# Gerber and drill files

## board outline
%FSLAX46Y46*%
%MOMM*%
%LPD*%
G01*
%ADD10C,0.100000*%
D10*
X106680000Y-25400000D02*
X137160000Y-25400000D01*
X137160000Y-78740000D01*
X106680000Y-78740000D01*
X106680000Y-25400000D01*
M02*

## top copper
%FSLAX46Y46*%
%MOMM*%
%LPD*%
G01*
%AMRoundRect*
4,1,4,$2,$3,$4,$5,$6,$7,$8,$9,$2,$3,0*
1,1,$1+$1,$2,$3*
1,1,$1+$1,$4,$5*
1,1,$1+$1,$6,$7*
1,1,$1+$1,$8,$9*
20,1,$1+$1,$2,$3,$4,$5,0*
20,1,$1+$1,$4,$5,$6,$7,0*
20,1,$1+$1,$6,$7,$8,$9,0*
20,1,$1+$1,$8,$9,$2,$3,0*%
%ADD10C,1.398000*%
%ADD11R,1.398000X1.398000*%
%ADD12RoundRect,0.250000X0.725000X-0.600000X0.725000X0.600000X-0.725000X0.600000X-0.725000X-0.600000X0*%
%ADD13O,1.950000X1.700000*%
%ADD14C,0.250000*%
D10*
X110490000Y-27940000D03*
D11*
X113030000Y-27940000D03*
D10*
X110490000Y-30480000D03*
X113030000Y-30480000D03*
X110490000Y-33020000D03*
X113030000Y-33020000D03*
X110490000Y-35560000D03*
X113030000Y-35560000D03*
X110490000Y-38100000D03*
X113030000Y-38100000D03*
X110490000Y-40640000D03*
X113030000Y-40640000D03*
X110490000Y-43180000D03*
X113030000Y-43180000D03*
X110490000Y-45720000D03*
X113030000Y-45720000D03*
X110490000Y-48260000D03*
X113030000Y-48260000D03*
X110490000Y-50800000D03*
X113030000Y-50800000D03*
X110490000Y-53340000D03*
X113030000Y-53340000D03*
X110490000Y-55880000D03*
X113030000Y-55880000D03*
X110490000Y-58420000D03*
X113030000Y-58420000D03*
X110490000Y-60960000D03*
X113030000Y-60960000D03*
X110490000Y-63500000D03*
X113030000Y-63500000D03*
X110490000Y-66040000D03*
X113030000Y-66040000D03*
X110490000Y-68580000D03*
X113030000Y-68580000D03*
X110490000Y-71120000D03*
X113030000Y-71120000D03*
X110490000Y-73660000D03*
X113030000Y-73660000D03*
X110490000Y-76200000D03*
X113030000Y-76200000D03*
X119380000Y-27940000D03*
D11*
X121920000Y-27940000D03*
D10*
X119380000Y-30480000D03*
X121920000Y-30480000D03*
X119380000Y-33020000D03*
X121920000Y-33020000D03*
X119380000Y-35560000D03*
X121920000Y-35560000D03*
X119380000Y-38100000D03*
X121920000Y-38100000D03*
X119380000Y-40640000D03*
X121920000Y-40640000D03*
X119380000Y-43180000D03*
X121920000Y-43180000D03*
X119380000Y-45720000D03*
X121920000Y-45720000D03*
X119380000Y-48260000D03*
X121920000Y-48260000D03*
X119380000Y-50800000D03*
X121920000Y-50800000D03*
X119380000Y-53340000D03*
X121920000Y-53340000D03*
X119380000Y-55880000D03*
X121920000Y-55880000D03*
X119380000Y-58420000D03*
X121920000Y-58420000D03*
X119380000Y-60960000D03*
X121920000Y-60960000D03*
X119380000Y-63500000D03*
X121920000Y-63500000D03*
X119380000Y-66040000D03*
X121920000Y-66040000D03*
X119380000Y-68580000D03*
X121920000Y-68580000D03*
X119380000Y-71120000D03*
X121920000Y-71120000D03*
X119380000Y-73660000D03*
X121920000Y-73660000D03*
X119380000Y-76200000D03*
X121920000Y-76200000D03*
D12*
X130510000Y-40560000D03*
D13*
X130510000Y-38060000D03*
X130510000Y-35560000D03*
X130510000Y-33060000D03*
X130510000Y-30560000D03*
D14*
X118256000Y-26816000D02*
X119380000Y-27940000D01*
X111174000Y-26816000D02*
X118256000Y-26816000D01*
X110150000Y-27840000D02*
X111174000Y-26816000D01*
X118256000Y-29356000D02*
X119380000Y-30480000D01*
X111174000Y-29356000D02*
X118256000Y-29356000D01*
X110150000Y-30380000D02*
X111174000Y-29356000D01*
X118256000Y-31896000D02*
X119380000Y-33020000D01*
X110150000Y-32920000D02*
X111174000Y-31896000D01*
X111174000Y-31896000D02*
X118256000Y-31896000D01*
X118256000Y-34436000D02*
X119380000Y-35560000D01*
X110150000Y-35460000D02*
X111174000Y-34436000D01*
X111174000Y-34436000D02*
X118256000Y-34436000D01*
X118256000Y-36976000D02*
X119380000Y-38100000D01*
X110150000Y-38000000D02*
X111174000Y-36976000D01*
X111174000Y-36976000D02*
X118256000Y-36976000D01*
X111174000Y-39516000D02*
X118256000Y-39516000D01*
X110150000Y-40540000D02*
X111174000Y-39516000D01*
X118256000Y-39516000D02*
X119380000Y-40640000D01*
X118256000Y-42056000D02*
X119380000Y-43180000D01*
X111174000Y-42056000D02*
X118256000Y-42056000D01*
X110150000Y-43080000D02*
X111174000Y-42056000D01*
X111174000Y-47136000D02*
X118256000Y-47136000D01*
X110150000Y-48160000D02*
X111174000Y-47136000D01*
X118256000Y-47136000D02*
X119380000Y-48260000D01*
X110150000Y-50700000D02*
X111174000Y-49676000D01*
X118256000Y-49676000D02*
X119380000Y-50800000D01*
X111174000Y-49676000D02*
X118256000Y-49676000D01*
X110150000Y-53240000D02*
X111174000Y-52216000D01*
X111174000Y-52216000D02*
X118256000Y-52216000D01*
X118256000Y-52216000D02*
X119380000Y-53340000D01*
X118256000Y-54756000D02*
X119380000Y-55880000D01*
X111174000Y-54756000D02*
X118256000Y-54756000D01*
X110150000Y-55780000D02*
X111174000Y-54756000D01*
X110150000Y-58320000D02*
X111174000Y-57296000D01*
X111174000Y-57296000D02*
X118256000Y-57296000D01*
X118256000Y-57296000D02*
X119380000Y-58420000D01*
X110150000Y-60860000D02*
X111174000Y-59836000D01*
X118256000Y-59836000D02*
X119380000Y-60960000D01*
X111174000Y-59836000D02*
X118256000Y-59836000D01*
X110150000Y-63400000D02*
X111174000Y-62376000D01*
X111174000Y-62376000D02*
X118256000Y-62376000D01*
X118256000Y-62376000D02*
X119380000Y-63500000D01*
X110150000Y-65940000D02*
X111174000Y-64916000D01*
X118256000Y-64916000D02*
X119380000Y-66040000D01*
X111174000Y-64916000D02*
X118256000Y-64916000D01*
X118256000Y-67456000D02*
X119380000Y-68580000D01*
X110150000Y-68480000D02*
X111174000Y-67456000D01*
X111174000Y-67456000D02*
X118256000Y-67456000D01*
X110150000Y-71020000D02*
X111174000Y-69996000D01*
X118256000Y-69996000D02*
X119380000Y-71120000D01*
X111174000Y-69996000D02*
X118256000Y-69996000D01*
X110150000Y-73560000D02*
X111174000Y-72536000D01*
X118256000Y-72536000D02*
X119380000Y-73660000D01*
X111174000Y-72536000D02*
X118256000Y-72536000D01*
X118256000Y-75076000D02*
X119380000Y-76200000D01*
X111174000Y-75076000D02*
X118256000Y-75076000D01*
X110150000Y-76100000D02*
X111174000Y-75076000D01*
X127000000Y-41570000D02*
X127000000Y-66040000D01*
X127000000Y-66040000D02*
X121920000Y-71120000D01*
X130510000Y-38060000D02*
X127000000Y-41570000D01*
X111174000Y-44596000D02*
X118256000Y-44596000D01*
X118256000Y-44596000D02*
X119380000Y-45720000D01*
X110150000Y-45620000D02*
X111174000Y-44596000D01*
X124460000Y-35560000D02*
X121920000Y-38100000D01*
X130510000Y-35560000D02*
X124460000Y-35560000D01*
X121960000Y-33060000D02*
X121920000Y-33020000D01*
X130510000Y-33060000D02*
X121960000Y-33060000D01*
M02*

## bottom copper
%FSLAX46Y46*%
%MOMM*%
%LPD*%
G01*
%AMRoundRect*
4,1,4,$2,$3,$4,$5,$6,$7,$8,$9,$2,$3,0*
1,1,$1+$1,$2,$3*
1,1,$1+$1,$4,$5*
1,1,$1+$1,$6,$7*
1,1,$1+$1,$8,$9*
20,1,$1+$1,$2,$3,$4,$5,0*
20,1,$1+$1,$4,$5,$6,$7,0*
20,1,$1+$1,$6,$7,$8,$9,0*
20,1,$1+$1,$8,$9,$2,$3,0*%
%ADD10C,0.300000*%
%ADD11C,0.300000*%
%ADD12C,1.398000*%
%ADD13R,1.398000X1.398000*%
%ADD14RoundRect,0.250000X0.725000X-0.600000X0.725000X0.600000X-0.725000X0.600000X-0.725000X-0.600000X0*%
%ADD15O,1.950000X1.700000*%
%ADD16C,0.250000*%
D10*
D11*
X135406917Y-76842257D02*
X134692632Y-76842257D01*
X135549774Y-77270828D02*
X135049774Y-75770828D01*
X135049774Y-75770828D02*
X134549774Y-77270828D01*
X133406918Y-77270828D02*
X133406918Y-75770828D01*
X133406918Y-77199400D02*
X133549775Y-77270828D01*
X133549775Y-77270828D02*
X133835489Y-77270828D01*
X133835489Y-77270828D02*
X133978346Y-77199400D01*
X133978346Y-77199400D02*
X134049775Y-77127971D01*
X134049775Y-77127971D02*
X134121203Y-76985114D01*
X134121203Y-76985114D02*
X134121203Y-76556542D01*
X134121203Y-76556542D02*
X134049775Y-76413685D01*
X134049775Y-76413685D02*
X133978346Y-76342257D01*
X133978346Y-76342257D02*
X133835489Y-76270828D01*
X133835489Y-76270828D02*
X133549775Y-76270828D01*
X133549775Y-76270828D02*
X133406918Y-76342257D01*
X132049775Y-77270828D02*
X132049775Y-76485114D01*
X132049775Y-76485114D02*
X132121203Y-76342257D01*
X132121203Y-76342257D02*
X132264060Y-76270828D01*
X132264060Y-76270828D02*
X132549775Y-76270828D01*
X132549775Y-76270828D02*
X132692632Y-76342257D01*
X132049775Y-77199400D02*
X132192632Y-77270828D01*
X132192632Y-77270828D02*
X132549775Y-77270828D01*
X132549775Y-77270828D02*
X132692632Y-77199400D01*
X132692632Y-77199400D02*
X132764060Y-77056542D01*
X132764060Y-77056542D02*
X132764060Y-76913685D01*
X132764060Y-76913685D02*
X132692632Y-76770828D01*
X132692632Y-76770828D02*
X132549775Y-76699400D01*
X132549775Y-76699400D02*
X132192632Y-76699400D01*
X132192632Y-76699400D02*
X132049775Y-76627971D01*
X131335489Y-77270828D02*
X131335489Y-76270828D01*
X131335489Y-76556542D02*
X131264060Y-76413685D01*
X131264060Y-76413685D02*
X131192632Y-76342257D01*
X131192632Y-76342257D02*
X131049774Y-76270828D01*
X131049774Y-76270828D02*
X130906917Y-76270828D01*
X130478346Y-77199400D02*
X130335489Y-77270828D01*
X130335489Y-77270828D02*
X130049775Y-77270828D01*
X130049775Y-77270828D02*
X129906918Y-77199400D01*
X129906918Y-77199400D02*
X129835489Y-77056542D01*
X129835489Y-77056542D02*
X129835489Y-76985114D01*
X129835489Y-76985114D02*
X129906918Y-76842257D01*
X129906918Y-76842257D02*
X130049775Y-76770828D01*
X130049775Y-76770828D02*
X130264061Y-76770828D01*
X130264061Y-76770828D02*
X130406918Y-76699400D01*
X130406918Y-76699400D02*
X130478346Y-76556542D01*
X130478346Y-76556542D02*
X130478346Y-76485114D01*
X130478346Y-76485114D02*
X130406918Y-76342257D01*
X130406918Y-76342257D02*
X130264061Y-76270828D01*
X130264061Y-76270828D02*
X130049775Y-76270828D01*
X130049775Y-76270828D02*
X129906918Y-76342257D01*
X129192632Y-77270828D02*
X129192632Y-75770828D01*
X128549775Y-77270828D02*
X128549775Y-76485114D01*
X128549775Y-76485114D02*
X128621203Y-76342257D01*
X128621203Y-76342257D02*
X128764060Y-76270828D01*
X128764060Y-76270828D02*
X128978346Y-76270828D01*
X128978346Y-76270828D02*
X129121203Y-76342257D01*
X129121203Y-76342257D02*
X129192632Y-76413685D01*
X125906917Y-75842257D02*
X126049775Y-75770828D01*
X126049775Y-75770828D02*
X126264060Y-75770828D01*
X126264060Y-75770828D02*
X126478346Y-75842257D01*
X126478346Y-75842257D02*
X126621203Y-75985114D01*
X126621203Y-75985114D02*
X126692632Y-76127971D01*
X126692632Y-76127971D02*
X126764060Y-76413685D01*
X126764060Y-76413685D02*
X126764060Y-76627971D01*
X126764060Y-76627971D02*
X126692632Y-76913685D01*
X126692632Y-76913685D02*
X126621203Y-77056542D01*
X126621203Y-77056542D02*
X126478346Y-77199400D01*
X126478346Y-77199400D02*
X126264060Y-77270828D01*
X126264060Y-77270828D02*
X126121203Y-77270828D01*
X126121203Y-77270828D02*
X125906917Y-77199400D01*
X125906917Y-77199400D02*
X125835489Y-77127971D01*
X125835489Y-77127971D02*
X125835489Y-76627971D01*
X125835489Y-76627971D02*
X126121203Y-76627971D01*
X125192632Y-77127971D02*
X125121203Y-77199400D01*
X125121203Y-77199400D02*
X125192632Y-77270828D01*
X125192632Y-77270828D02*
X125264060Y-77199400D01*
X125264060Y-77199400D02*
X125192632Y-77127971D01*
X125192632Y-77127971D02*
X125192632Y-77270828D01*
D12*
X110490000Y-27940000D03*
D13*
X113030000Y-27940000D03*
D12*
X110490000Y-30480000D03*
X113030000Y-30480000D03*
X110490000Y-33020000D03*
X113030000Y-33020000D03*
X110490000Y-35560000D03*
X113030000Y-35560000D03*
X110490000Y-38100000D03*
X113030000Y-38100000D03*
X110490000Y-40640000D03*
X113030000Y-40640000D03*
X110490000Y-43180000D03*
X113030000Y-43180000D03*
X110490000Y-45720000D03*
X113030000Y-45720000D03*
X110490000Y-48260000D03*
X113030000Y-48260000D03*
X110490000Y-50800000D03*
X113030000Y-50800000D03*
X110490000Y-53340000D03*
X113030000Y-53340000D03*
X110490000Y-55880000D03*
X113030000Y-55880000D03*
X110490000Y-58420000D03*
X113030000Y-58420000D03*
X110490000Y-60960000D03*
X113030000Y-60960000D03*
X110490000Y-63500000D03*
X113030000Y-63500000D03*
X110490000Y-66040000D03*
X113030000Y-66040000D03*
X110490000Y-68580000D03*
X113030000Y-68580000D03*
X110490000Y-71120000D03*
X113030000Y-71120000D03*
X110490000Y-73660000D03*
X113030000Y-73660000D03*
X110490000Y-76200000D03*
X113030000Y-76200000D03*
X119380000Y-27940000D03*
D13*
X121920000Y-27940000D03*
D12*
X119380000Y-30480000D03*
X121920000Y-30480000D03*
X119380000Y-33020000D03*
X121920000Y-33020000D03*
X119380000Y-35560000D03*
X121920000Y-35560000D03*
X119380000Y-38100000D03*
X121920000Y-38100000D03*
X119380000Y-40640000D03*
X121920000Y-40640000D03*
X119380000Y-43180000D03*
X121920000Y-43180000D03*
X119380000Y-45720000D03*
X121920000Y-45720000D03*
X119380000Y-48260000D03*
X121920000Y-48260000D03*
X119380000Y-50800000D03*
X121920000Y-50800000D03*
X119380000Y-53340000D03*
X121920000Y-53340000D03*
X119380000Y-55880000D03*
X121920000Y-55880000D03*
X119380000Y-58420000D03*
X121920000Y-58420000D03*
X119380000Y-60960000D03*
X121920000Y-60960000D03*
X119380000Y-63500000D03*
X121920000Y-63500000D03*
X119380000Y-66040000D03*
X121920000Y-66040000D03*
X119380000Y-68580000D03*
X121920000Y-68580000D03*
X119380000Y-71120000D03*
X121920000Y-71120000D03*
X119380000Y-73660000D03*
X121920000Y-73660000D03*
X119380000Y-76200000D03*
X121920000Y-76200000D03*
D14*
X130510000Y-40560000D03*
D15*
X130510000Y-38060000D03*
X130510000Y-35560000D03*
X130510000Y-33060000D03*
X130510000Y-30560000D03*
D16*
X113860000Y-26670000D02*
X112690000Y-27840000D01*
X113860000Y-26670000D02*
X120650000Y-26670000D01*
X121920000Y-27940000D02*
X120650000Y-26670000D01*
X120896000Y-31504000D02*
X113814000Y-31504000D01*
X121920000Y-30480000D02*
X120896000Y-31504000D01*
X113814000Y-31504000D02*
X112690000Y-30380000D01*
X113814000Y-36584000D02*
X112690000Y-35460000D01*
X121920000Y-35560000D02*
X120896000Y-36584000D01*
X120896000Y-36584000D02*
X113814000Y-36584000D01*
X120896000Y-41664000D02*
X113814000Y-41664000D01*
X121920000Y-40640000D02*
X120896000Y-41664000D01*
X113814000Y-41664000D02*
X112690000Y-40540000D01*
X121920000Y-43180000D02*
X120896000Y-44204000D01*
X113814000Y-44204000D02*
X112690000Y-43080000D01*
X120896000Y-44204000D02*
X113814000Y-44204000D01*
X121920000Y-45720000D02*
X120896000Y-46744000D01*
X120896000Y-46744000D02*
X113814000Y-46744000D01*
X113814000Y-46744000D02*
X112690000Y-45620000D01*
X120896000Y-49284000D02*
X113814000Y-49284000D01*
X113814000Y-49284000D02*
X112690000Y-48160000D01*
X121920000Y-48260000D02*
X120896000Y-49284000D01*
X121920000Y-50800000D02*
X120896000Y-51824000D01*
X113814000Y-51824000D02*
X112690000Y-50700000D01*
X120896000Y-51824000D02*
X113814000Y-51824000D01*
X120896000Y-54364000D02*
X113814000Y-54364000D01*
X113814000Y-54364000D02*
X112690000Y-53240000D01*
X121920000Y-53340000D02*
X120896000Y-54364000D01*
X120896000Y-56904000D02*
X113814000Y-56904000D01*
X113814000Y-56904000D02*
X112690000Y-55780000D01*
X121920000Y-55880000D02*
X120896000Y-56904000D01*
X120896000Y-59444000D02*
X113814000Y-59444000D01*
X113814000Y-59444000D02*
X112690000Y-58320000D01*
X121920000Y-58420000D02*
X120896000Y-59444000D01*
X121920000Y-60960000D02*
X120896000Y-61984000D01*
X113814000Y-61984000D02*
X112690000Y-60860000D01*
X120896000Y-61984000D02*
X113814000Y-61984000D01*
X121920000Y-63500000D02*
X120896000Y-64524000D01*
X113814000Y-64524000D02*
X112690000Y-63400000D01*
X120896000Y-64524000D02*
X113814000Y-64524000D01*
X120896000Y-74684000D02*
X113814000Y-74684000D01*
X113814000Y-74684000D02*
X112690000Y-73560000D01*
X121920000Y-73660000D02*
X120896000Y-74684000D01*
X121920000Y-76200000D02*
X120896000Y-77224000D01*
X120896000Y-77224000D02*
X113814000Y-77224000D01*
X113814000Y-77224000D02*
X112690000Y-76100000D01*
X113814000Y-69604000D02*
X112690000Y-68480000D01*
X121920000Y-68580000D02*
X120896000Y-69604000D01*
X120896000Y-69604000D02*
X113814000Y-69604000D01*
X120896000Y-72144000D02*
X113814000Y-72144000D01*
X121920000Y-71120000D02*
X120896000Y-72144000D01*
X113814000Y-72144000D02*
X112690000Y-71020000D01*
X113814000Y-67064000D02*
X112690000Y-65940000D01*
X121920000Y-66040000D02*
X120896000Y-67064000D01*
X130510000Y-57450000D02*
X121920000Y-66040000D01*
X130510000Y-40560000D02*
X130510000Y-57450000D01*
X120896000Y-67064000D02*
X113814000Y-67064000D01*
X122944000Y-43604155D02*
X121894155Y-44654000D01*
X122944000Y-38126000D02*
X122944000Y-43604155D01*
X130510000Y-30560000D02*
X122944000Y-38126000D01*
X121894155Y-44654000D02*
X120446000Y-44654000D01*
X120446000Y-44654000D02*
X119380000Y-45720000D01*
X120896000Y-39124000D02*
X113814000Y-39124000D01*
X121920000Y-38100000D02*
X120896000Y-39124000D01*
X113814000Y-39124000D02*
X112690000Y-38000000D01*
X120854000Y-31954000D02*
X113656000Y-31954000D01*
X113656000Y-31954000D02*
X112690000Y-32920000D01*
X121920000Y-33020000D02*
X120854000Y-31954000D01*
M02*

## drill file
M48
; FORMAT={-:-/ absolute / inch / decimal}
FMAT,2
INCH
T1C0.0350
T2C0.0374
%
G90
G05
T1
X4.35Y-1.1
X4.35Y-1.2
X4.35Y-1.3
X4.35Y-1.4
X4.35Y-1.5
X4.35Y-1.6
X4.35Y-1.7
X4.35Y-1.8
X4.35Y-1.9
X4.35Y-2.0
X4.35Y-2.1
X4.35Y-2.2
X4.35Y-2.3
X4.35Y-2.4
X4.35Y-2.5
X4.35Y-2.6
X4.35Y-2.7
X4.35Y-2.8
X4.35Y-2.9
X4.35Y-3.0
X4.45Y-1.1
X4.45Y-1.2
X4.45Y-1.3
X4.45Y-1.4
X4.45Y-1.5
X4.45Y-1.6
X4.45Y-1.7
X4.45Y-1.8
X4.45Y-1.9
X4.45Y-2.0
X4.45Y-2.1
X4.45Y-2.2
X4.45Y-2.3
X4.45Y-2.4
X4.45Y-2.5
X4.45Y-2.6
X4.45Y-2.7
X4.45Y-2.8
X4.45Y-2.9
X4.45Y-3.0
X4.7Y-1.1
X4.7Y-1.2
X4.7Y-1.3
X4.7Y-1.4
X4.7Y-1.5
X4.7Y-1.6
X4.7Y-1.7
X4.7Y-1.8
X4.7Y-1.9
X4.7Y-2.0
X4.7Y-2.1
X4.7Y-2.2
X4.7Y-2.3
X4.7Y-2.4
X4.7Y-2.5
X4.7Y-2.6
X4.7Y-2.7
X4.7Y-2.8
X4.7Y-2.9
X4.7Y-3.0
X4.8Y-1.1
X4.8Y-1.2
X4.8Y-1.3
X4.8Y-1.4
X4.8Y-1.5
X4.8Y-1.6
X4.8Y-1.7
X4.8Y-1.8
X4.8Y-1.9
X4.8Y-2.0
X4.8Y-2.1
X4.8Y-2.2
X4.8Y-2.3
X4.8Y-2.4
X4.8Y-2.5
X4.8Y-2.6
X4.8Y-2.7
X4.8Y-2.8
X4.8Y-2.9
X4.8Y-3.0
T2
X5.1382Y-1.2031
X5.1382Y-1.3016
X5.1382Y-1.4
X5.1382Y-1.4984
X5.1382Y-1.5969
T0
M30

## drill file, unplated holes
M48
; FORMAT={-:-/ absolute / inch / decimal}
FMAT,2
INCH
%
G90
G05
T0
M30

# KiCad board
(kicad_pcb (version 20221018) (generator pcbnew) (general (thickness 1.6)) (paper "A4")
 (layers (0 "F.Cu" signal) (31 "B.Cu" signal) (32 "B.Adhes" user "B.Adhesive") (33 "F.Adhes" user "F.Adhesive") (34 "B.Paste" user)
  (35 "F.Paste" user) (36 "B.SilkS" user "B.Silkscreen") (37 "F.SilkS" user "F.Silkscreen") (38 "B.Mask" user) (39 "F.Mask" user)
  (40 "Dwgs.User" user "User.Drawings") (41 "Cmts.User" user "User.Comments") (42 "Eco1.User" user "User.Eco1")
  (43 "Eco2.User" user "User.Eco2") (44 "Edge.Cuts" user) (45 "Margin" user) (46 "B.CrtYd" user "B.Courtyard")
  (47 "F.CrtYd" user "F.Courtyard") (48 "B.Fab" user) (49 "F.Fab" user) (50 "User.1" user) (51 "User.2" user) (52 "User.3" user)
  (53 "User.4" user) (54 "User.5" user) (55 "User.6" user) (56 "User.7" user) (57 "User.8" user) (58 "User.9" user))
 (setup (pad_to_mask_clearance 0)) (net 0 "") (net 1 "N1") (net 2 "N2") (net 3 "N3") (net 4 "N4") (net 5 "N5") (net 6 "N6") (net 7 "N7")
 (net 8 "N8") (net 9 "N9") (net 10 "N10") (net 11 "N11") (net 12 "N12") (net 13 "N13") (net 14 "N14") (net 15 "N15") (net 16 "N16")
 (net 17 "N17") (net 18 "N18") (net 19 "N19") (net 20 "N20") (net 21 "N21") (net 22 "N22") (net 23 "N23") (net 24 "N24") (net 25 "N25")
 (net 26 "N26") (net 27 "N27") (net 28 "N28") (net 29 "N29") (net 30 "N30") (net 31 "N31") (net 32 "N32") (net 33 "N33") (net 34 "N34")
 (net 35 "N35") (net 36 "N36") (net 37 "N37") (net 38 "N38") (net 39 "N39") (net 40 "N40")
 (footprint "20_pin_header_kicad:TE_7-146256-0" (layer "F.Cu") (at 111.76 52.07 -90)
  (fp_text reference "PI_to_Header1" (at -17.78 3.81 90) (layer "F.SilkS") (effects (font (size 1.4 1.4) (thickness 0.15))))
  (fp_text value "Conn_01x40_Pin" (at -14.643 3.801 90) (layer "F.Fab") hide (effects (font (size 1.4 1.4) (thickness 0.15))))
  (pad "1" thru_hole circle (at -24.13 1.27 270) (size 1.398 1.398) (drill 0.89) (layers "*.Cu" "*.Mask") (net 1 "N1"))
  (pad "2" thru_hole rect (at -24.13 -1.27 270) (size 1.398 1.398) (drill 0.89) (layers "*.Cu" "*.Mask") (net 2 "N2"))
  (pad "3" thru_hole circle (at -21.59 1.27 270) (size 1.398 1.398) (drill 0.89) (layers "*.Cu" "*.Mask") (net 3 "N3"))
  (pad "4" thru_hole circle (at -21.59 -1.27 270) (size 1.398 1.398) (drill 0.89) (layers "*.Cu" "*.Mask") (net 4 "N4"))
  (pad "5" thru_hole circle (at -19.05 1.27 270) (size 1.398 1.398) (drill 0.89) (layers "*.Cu" "*.Mask") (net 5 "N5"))
  (pad "6" thru_hole circle (at -19.05 -1.27 270) (size 1.398 1.398) (drill 0.89) (layers "*.Cu" "*.Mask") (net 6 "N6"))
  (pad "7" thru_hole circle (at -16.51 1.27 270) (size 1.398 1.398) (drill 0.89) (layers "*.Cu" "*.Mask") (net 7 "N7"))
  (pad "8" thru_hole circle (at -16.51 -1.27 270) (size 1.398 1.398) (drill 0.89) (layers "*.Cu" "*.Mask") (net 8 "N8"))
  (pad "9" thru_hole circle (at -13.97 1.27 270) (size 1.398 1.398) (drill 0.89) (layers "*.Cu" "*.Mask") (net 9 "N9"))
  (pad "10" thru_hole circle (at -13.97 -1.27 270) (size 1.398 1.398) (drill 0.89) (layers "*.Cu" "*.Mask") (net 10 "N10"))
  (pad "11" thru_hole circle (at -11.43 1.27 270) (size 1.398 1.398) (drill 0.89) (layers "*.Cu" "*.Mask") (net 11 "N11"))
  (pad "12" thru_hole circle (at -11.43 -1.27 270) (size 1.398 1.398) (drill 0.89) (layers "*.Cu" "*.Mask") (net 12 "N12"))
  (pad "13" thru_hole circle (at -8.89 1.27 270) (size 1.398 1.398) (drill 0.89) (layers "*.Cu" "*.Mask") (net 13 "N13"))
  (pad "14" thru_hole circle (at -8.89 -1.27 270) (size 1.398 1.398) (drill 0.89) (layers "*.Cu" "*.Mask") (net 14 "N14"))
  (pad "15" thru_hole circle (at -6.35 1.27 270) (size 1.398 1.398) (drill 0.89) (layers "*.Cu" "*.Mask") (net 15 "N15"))
  (pad "16" thru_hole circle (at -6.35 -1.27 270) (size 1.398 1.398) (drill 0.89) (layers "*.Cu" "*.Mask") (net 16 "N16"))
  (pad "17" thru_hole circle (at -3.81 1.27 270) (size 1.398 1.398) (drill 0.89) (layers "*.Cu" "*.Mask") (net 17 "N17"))
  (pad "18" thru_hole circle (at -3.81 -1.27 270) (size 1.398 1.398) (drill 0.89) (layers "*.Cu" "*.Mask") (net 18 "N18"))
  (pad "19" thru_hole circle (at -1.27 1.27 270) (size 1.398 1.398) (drill 0.89) (layers "*.Cu" "*.Mask") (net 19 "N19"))
  (pad "20" thru_hole circle (at -1.27 -1.27 270) (size 1.398 1.398) (drill 0.89) (layers "*.Cu" "*.Mask") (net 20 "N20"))
  (pad "21" thru_hole circle (at 1.27 1.27 270) (size 1.398 1.398) (drill 0.89) (layers "*.Cu" "*.Mask") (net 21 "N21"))
  (pad "22" thru_hole circle (at 1.27 -1.27 270) (size 1.398 1.398) (drill 0.89) (layers "*.Cu" "*.Mask") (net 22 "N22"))
  (pad "23" thru_hole circle (at 3.81 1.27 270) (size 1.398 1.398) (drill 0.89) (layers "*.Cu" "*.Mask") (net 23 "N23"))
  (pad "24" thru_hole circle (at 3.81 -1.27 270) (size 1.398 1.398) (drill 0.89) (layers "*.Cu" "*.Mask") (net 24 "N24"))
  (pad "25" thru_hole circle (at 6.35 1.27 270) (size 1.398 1.398) (drill 0.89) (layers "*.Cu" "*.Mask") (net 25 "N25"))
  (pad "26" thru_hole circle (at 6.35 -1.27 270) (size 1.398 1.398) (drill 0.89) (layers "*.Cu" "*.Mask") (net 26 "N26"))
  (pad "27" thru_hole circle (at 8.89 1.27 270) (size 1.398 1.398) (drill 0.89) (layers "*.Cu" "*.Mask") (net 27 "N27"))
  (pad "28" thru_hole circle (at 8.89 -1.27 270) (size 1.398 1.398) (drill 0.89) (layers "*.Cu" "*.Mask") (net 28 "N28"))
  (pad "29" thru_hole circle (at 11.43 1.27 270) (size 1.398 1.398) (drill 0.89) (layers "*.Cu" "*.Mask") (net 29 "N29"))
  (pad "30" thru_hole circle (at 11.43 -1.27 270) (size 1.398 1.398) (drill 0.89) (layers "*.Cu" "*.Mask") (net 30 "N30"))
  (pad "31" thru_hole circle (at 13.97 1.27 270) (size 1.398 1.398) (drill 0.89) (layers "*.Cu" "*.Mask") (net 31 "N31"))
  (pad "32" thru_hole circle (at 13.97 -1.27 270) (size 1.398 1.398) (drill 0.89) (layers "*.Cu" "*.Mask") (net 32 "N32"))
  (pad "33" thru_hole circle (at 16.51 1.27 270) (size 1.398 1.398) (drill 0.89) (layers "*.Cu" "*.Mask") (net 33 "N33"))
  (pad "34" thru_hole circle (at 16.51 -1.27 270) (size 1.398 1.398) (drill 0.89) (layers "*.Cu" "*.Mask") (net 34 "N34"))
  (pad "35" thru_hole circle (at 19.05 1.27 270) (size 1.398 1.398) (drill 0.89) (layers "*.Cu" "*.Mask") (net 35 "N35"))
  (pad "36" thru_hole circle (at 19.05 -1.27 270) (size 1.398 1.398) (drill 0.89) (layers "*.Cu" "*.Mask") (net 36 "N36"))
  (pad "37" thru_hole circle (at 21.59 1.27 270) (size 1.398 1.398) (drill 0.89) (layers "*.Cu" "*.Mask") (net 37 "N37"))
  (pad "38" thru_hole circle (at 21.59 -1.27 270) (size 1.398 1.398) (drill 0.89) (layers "*.Cu" "*.Mask") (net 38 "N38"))
  (pad "39" thru_hole circle (at 24.13 1.27 270) (size 1.398 1.398) (drill 0.89) (layers "*.Cu" "*.Mask") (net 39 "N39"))
  (pad "40" thru_hole circle (at 24.13 -1.27 270) (size 1.398 1.398) (drill 0.89) (layers "*.Cu" "*.Mask") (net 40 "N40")))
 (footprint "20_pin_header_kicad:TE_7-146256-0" (layer "F.Cu") (at 120.65 52.07 -90)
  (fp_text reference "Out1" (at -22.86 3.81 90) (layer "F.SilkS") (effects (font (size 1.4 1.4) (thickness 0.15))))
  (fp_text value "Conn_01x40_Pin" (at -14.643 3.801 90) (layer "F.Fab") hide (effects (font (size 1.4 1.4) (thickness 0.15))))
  (pad "1" thru_hole circle (at -24.13 1.27 270) (size 1.398 1.398) (drill 0.89) (layers "*.Cu" "*.Mask") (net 1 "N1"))
  (pad "2" thru_hole rect (at -24.13 -1.27 270) (size 1.398 1.398) (drill 0.89) (layers "*.Cu" "*.Mask") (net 2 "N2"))
  (pad "3" thru_hole circle (at -21.59 1.27 270) (size 1.398 1.398) (drill 0.89) (layers "*.Cu" "*.Mask") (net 3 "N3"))
  (pad "4" thru_hole circle (at -21.59 -1.27 270) (size 1.398 1.398) (drill 0.89) (layers "*.Cu" "*.Mask") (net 4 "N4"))
  (pad "5" thru_hole circle (at -19.05 1.27 270) (size 1.398 1.398) (drill 0.89) (layers "*.Cu" "*.Mask") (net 5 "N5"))
  (pad "6" thru_hole circle (at -19.05 -1.27 270) (size 1.398 1.398) (drill 0.89) (layers "*.Cu" "*.Mask") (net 6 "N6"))
  (pad "7" thru_hole circle (at -16.51 1.27 270) (size 1.398 1.398) (drill 0.89) (layers "*.Cu" "*.Mask") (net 7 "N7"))
  (pad "8" thru_hole circle (at -16.51 -1.27 270) (size 1.398 1.398) (drill 0.89) (layers "*.Cu" "*.Mask") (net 8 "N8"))
  (pad "9" thru_hole circle (at -13.97 1.27 270) (size 1.398 1.398) (drill 0.89) (layers "*.Cu" "*.Mask") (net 9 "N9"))
  (pad "10" thru_hole circle (at -13.97 -1.27 270) (size 1.398 1.398) (drill 0.89) (layers "*.Cu" "*.Mask") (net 10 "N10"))
  (pad "11" thru_hole circle (at -11.43 1.27 270) (size 1.398 1.398) (drill 0.89) (layers "*.Cu" "*.Mask") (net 11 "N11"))
  (pad "12" thru_hole circle (at -11.43 -1.27 270) (size 1.398 1.398) (drill 0.89) (layers "*.Cu" "*.Mask") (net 12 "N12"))
  (pad "13" thru_hole circle (at -8.89 1.27 270) (size 1.398 1.398) (drill 0.89) (layers "*.Cu" "*.Mask") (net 13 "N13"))
  (pad "14" thru_hole circle (at -8.89 -1.27 270) (size 1.398 1.398) (drill 0.89) (layers "*.Cu" "*.Mask") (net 14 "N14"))
  (pad "15" thru_hole circle (at -6.35 1.27 270) (size 1.398 1.398) (drill 0.89) (layers "*.Cu" "*.Mask") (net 15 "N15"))
  (pad "16" thru_hole circle (at -6.35 -1.27 270) (size 1.398 1.398) (drill 0.89) (layers "*.Cu" "*.Mask") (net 16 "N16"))
  (pad "17" thru_hole circle (at -3.81 1.27 270) (size 1.398 1.398) (drill 0.89) (layers "*.Cu" "*.Mask") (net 17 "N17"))
  (pad "18" thru_hole circle (at -3.81 -1.27 270) (size 1.398 1.398) (drill 0.89) (layers "*.Cu" "*.Mask") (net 18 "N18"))
  (pad "19" thru_hole circle (at -1.27 1.27 270) (size 1.398 1.398) (drill 0.89) (layers "*.Cu" "*.Mask") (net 19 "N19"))
  (pad "20" thru_hole circle (at -1.27 -1.27 270) (size 1.398 1.398) (drill 0.89) (layers "*.Cu" "*.Mask") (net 20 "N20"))
  (pad "21" thru_hole circle (at 1.27 1.27 270) (size 1.398 1.398) (drill 0.89) (layers "*.Cu" "*.Mask") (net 21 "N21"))
  (pad "22" thru_hole circle (at 1.27 -1.27 270) (size 1.398 1.398) (drill 0.89) (layers "*.Cu" "*.Mask") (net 22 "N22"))
  (pad "23" thru_hole circle (at 3.81 1.27 270) (size 1.398 1.398) (drill 0.89) (layers "*.Cu" "*.Mask") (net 23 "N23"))
  (pad "24" thru_hole circle (at 3.81 -1.27 270) (size 1.398 1.398) (drill 0.89) (layers "*.Cu" "*.Mask") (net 24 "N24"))
  (pad "25" thru_hole circle (at 6.35 1.27 270) (size 1.398 1.398) (drill 0.89) (layers "*.Cu" "*.Mask") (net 25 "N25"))
  (pad "26" thru_hole circle (at 6.35 -1.27 270) (size 1.398 1.398) (drill 0.89) (layers "*.Cu" "*.Mask") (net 26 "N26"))
  (pad "27" thru_hole circle (at 8.89 1.27 270) (size 1.398 1.398) (drill 0.89) (layers "*.Cu" "*.Mask") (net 27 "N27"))
  (pad "28" thru_hole circle (at 8.89 -1.27 270) (size 1.398 1.398) (drill 0.89) (layers "*.Cu" "*.Mask") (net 28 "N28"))
  (pad "29" thru_hole circle (at 11.43 1.27 270) (size 1.398 1.398) (drill 0.89) (layers "*.Cu" "*.Mask") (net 29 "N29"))
  (pad "30" thru_hole circle (at 11.43 -1.27 270) (size 1.398 1.398) (drill 0.89) (layers "*.Cu" "*.Mask") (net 30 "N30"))
  (pad "31" thru_hole circle (at 13.97 1.27 270) (size 1.398 1.398) (drill 0.89) (layers "*.Cu" "*.Mask") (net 31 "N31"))
  (pad "32" thru_hole circle (at 13.97 -1.27 270) (size 1.398 1.398) (drill 0.89) (layers "*.Cu" "*.Mask") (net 32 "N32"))
  (pad "33" thru_hole circle (at 16.51 1.27 270) (size 1.398 1.398) (drill 0.89) (layers "*.Cu" "*.Mask") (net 33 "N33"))
  (pad "34" thru_hole circle (at 16.51 -1.27 270) (size 1.398 1.398) (drill 0.89) (layers "*.Cu" "*.Mask") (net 34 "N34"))
  (pad "35" thru_hole circle (at 19.05 1.27 270) (size 1.398 1.398) (drill 0.89) (layers "*.Cu" "*.Mask") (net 35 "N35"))
  (pad "36" thru_hole circle (at 19.05 -1.27 270) (size 1.398 1.398) (drill 0.89) (layers "*.Cu" "*.Mask") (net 36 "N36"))
  (pad "37" thru_hole circle (at 21.59 1.27 270) (size 1.398 1.398) (drill 0.89) (layers "*.Cu" "*.Mask") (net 37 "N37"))
  (pad "38" thru_hole circle (at 21.59 -1.27 270) (size 1.398 1.398) (drill 0.89) (layers "*.Cu" "*.Mask") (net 38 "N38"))
  (pad "39" thru_hole circle (at 24.13 1.27 270) (size 1.398 1.398) (drill 0.89) (layers "*.Cu" "*.Mask") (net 39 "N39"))
  (pad "40" thru_hole circle (at 24.13 -1.27 270) (size 1.398 1.398) (drill 0.89) (layers "*.Cu" "*.Mask") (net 40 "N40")))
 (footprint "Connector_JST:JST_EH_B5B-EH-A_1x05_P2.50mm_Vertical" (layer "F.Cu") (at 130.51 40.56 90)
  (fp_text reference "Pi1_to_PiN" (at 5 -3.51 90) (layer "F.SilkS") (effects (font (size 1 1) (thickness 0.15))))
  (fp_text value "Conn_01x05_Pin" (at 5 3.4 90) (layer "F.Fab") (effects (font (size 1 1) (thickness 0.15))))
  (pad "1" thru_hole roundrect (at 0 0 90) (size 1.7 1.95) (drill 0.95) (layers "*.Cu" "*.Mask") (roundrect_rratio 0.1470588235)
   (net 32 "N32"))
  (pad "2" thru_hole oval (at 2.5 0 90) (size 1.7 1.95) (drill 0.95) (layers "*.Cu" "*.Mask") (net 36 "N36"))
  (pad "3" thru_hole oval (at 5 0 90) (size 1.7 1.95) (drill 0.95) (layers "*.Cu" "*.Mask") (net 10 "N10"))
  (pad "4" thru_hole oval (at 7.5 0 90) (size 1.7 1.95) (drill 0.95) (layers "*.Cu" "*.Mask") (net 6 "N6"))
  (pad "5" thru_hole oval (at 10 0 90) (size 1.7 1.95) (drill 0.95) (layers "*.Cu" "*.Mask") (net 15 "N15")))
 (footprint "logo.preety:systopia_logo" (layer "F.Cu") (at 130.81 68.58)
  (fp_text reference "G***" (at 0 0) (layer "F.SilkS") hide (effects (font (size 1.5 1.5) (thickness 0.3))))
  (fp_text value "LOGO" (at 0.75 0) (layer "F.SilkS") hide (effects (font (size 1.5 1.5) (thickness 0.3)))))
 (gr_rect (start 106.68 25.4) (end 137.16 78.74) (stroke (width 0.1) (type default)) (fill none) (layer "Edge.Cuts"))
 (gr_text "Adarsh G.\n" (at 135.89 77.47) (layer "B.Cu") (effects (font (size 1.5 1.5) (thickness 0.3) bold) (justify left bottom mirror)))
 (segment (start 118.256 26.816) (end 119.38 27.94) (width 0.25) (layer "F.Cu") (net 1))
 (segment (start 111.174 26.816) (end 118.256 26.816) (width 0.25) (layer "F.Cu") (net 1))
 (segment (start 110.15 27.84) (end 111.174 26.816) (width 0.25) (layer "F.Cu") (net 1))
 (segment (start 113.86 26.67) (end 112.69 27.84) (width 0.25) (layer "B.Cu") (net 2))
 (segment (start 113.86 26.67) (end 120.65 26.67) (width 0.25) (layer "B.Cu") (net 2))
 (segment (start 121.92 27.94) (end 120.65 26.67) (width 0.25) (layer "B.Cu") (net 2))
 (segment (start 118.256 29.356) (end 119.38 30.48) (width 0.25) (layer "F.Cu") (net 3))
 (segment (start 111.174 29.356) (end 118.256 29.356) (width 0.25) (layer "F.Cu") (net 3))
 (segment (start 110.15 30.38) (end 111.174 29.356) (width 0.25) (layer "F.Cu") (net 3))
 (segment (start 120.896 31.504) (end 113.814 31.504) (width 0.25) (layer "B.Cu") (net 4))
 (segment (start 121.92 30.48) (end 120.896 31.504) (width 0.25) (layer "B.Cu") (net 4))
 (segment (start 113.814 31.504) (end 112.69 30.38) (width 0.25) (layer "B.Cu") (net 4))
 (segment (start 118.256 31.896) (end 119.38 33.02) (width 0.25) (layer "F.Cu") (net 5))
 (segment (start 110.15 32.92) (end 111.174 31.896) (width 0.25) (layer "F.Cu") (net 5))
 (segment (start 111.174 31.896) (end 118.256 31.896) (width 0.25) (layer "F.Cu") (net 5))
 (segment (start 118.256 34.436) (end 119.38 35.56) (width 0.25) (layer "F.Cu") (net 7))
 (segment (start 110.15 35.46) (end 111.174 34.436) (width 0.25) (layer "F.Cu") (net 7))
 (segment (start 111.174 34.436) (end 118.256 34.436) (width 0.25) (layer "F.Cu") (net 7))
 (segment (start 113.814 36.584) (end 112.69 35.46) (width 0.25) (layer "B.Cu") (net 8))
 (segment (start 121.92 35.56) (end 120.896 36.584) (width 0.25) (layer "B.Cu") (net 8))
 (segment (start 120.896 36.584) (end 113.814 36.584) (width 0.25) (layer "B.Cu") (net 8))
 (segment (start 118.256 36.976) (end 119.38 38.1) (width 0.25) (layer "F.Cu") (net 9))
 (segment (start 110.15 38) (end 111.174 36.976) (width 0.25) (layer "F.Cu") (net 9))
 (segment (start 111.174 36.976) (end 118.256 36.976) (width 0.25) (layer "F.Cu") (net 9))
 (segment (start 111.174 39.516) (end 118.256 39.516) (width 0.25) (layer "F.Cu") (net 11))
 (segment (start 110.15 40.54) (end 111.174 39.516) (width 0.25) (layer "F.Cu") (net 11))
 (segment (start 118.256 39.516) (end 119.38 40.64) (width 0.25) (layer "F.Cu") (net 11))
 (segment (start 120.896 41.664) (end 113.814 41.664) (width 0.25) (layer "B.Cu") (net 12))
 (segment (start 121.92 40.64) (end 120.896 41.664) (width 0.25) (layer "B.Cu") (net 12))
 (segment (start 113.814 41.664) (end 112.69 40.54) (width 0.25) (layer "B.Cu") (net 12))
 (segment (start 118.256 42.056) (end 119.38 43.18) (width 0.25) (layer "F.Cu") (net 13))
 (segment (start 111.174 42.056) (end 118.256 42.056) (width 0.25) (layer "F.Cu") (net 13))
 (segment (start 110.15 43.08) (end 111.174 42.056) (width 0.25) (layer "F.Cu") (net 13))
 (segment (start 121.92 43.18) (end 120.896 44.204) (width 0.25) (layer "B.Cu") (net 14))
 (segment (start 113.814 44.204) (end 112.69 43.08) (width 0.25) (layer "B.Cu") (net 14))
 (segment (start 120.896 44.204) (end 113.814 44.204) (width 0.25) (layer "B.Cu") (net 14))
 (segment (start 121.92 45.72) (end 120.896 46.744) (width 0.25) (layer "B.Cu") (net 16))
 (segment (start 120.896 46.744) (end 113.814 46.744) (width 0.25) (layer "B.Cu") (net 16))
 (segment (start 113.814 46.744) (end 112.69 45.62) (width 0.25) (layer "B.Cu") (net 16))
 (segment (start 111.174 47.136) (end 118.256 47.136) (width 0.25) (layer "F.Cu") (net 17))
 (segment (start 110.15 48.16) (end 111.174 47.136) (width 0.25) (layer "F.Cu") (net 17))
 (segment (start 118.256 47.136) (end 119.38 48.26) (width 0.25) (layer "F.Cu") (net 17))
 (segment (start 120.896 49.284) (end 113.814 49.284) (width 0.25) (layer "B.Cu") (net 18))
 (segment (start 113.814 49.284) (end 112.69 48.16) (width 0.25) (layer "B.Cu") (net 18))
 (segment (start 121.92 48.26) (end 120.896 49.284) (width 0.25) (layer "B.Cu") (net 18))
 (segment (start 110.15 50.7) (end 111.174 49.676) (width 0.25) (layer "F.Cu") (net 19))
 (segment (start 118.256 49.676) (end 119.38 50.8) (width 0.25) (layer "F.Cu") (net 19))
 (segment (start 111.174 49.676) (end 118.256 49.676) (width 0.25) (layer "F.Cu") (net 19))
 (segment (start 121.92 50.8) (end 120.896 51.824) (width 0.25) (layer "B.Cu") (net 20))
 (segment (start 113.814 51.824) (end 112.69 50.7) (width 0.25) (layer "B.Cu") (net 20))
 (segment (start 120.896 51.824) (end 113.814 51.824) (width 0.25) (layer "B.Cu") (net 20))
 (segment (start 110.15 53.24) (end 111.174 52.216) (width 0.25) (layer "F.Cu") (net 21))
 (segment (start 111.174 52.216) (end 118.256 52.216) (width 0.25) (layer "F.Cu") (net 21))
 (segment (start 118.256 52.216) (end 119.38 53.34) (width 0.25) (layer "F.Cu") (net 21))
 (segment (start 120.896 54.364) (end 113.814 54.364) (width 0.25) (layer "B.Cu") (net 22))
 (segment (start 113.814 54.364) (end 112.69 53.24) (width 0.25) (layer "B.Cu") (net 22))
 (segment (start 121.92 53.34) (end 120.896 54.364) (width 0.25) (layer "B.Cu") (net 22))
 (segment (start 118.256 54.756) (end 119.38 55.88) (width 0.25) (layer "F.Cu") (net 23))
 (segment (start 111.174 54.756) (end 118.256 54.756) (width 0.25) (layer "F.Cu") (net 23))
 (segment (start 110.15 55.78) (end 111.174 54.756) (width 0.25) (layer "F.Cu") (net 23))
 (segment (start 120.896 56.904) (end 113.814 56.904) (width 0.25) (layer "B.Cu") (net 24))
 (segment (start 113.814 56.904) (end 112.69 55.78) (width 0.25) (layer "B.Cu") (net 24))
 (segment (start 121.92 55.88) (end 120.896 56.904) (width 0.25) (layer "B.Cu") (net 24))
 (segment (start 110.15 58.32) (end 111.174 57.296) (width 0.25) (layer "F.Cu") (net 25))
 (segment (start 111.174 57.296) (end 118.256 57.296) (width 0.25) (layer "F.Cu") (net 25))
 (segment (start 118.256 57.296) (end 119.38 58.42) (width 0.25) (layer "F.Cu") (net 25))
 (segment (start 120.896 59.444) (end 113.814 59.444) (width 0.25) (layer "B.Cu") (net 26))
 (segment (start 113.814 59.444) (end 112.69 58.32) (width 0.25) (layer "B.Cu") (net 26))
 (segment (start 121.92 58.42) (end 120.896 59.444) (width 0.25) (layer "B.Cu") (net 26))
 (segment (start 110.15 60.86) (end 111.174 59.836) (width 0.25) (layer "F.Cu") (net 27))
 (segment (start 118.256 59.836) (end 119.38 60.96) (width 0.25) (layer "F.Cu") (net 27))
 (segment (start 111.174 59.836) (end 118.256 59.836) (width 0.25) (layer "F.Cu") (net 27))
 (segment (start 121.92 60.96) (end 120.896 61.984) (width 0.25) (layer "B.Cu") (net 28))
 (segment (start 113.814 61.984) (end 112.69 60.86) (width 0.25) (layer "B.Cu") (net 28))
 (segment (start 120.896 61.984) (end 113.814 61.984) (width 0.25) (layer "B.Cu") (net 28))
 (segment (start 110.15 63.4) (end 111.174 62.376) (width 0.25) (layer "F.Cu") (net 29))
 (segment (start 111.174 62.376) (end 118.256 62.376) (width 0.25) (layer "F.Cu") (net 29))
 (segment (start 118.256 62.376) (end 119.38 63.5) (width 0.25) (layer "F.Cu") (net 29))
 (segment (start 121.92 63.5) (end 120.896 64.524) (width 0.25) (layer "B.Cu") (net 30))
 (segment (start 113.814 64.524) (end 112.69 63.4) (width 0.25) (layer "B.Cu") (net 30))
 (segment (start 120.896 64.524) (end 113.814 64.524) (width 0.25) (layer "B.Cu") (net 30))
 (segment (start 110.15 65.94) (end 111.174 64.916) (width 0.25) (layer "F.Cu") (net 31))
 (segment (start 118.256 64.916) (end 119.38 66.04) (width 0.25) (layer "F.Cu") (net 31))
 (segment (start 111.174 64.916) (end 118.256 64.916) (width 0.25) (layer "F.Cu") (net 31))
 (segment (start 118.256 67.456) (end 119.38 68.58) (width 0.25) (layer "F.Cu") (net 33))
 (segment (start 110.15 68.48) (end 111.174 67.456) (width 0.25) (layer "F.Cu") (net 33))
 (segment (start 111.174 67.456) (end 118.256 67.456) (width 0.25) (layer "F.Cu") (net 33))
 (segment (start 110.15 71.02) (end 111.174 69.996) (width 0.25) (layer "F.Cu") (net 35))
 (segment (start 118.256 69.996) (end 119.38 71.12) (width 0.25) (layer "F.Cu") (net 35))
 (segment (start 111.174 69.996) (end 118.256 69.996) (width 0.25) (layer "F.Cu") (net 35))
 (segment (start 110.15 73.56) (end 111.174 72.536) (width 0.25) (layer "F.Cu") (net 37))
 (segment (start 118.256 72.536) (end 119.38 73.66) (width 0.25) (layer "F.Cu") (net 37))
 (segment (start 111.174 72.536) (end 118.256 72.536) (width 0.25) (layer "F.Cu") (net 37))
 (segment (start 120.896 74.684) (end 113.814 74.684) (width 0.25) (layer "B.Cu") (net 38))
 (segment (start 113.814 74.684) (end 112.69 73.56) (width 0.25) (layer "B.Cu") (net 38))
 (segment (start 121.92 73.66) (end 120.896 74.684) (width 0.25) (layer "B.Cu") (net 38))
 (segment (start 118.256 75.076) (end 119.38 76.2) (width 0.25) (layer "F.Cu") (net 39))
 (segment (start 111.174 75.076) (end 118.256 75.076) (width 0.25) (layer "F.Cu") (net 39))
 (segment (start 110.15 76.1) (end 111.174 75.076) (width 0.25) (layer "F.Cu") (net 39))
 (segment (start 121.92 76.2) (end 120.896 77.224) (width 0.25) (layer "B.Cu") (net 40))
 (segment (start 120.896 77.224) (end 113.814 77.224) (width 0.25) (layer "B.Cu") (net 40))
 (segment (start 113.814 77.224) (end 112.69 76.1) (width 0.25) (layer "B.Cu") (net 40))
 (segment (start 113.814 69.604) (end 112.69 68.48) (width 0.25) (layer "B.Cu") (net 34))
 (segment (start 121.92 68.58) (end 120.896 69.604) (width 0.25) (layer "B.Cu") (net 34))
 (segment (start 120.896 69.604) (end 113.814 69.604) (width 0.25) (layer "B.Cu") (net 34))
 (segment (start 127 41.57) (end 127 66.04) (width 0.25) (layer "F.Cu") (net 36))
 (segment (start 127 66.04) (end 121.92 71.12) (width 0.25) (layer "F.Cu") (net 36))
 (segment (start 130.51 38.06) (end 127 41.57) (width 0.25) (layer "F.Cu") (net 36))
 (segment (start 120.896 72.144) (end 113.814 72.144) (width 0.25) (layer "B.Cu") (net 36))
 (segment (start 121.92 71.12) (end 120.896 72.144) (width 0.25) (layer "B.Cu") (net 36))
 (segment (start 113.814 72.144) (end 112.69 71.02) (width 0.25) (layer "B.Cu") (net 36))
 (segment (start 113.814 67.064) (end 112.69 65.94) (width 0.25) (layer "B.Cu") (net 32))
 (segment (start 121.92 66.04) (end 120.896 67.064) (width 0.25) (layer "B.Cu") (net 32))
 (segment (start 130.51 57.45) (end 121.92 66.04) (width 0.25) (layer "B.Cu") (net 32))
 (segment (start 130.51 40.56) (end 130.51 57.45) (width 0.25) (layer "B.Cu") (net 32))
 (segment (start 120.896 67.064) (end 113.814 67.064) (width 0.25) (layer "B.Cu") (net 32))
 (segment (start 111.174 44.596) (end 118.256 44.596) (width 0.25) (layer "F.Cu") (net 15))
 (segment (start 118.256 44.596) (end 119.38 45.72) (width 0.25) (layer "F.Cu") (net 15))
 (segment (start 110.15 45.62) (end 111.174 44.596) (width 0.25) (layer "F.Cu") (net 15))
 (segment (start 122.944 43.604155) (end 121.894155 44.654) (width 0.25) (layer "B.Cu") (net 15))
 (segment (start 122.944 38.126) (end 122.944 43.604155) (width 0.25) (layer "B.Cu") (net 15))
 (segment (start 130.51 30.56) (end 122.944 38.126) (width 0.25) (layer "B.Cu") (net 15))
 (segment (start 121.894155 44.654) (end 120.446 44.654) (width 0.25) (layer "B.Cu") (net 15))
 (segment (start 120.446 44.654) (end 119.38 45.72) (width 0.25) (layer "B.Cu") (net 15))
 (segment (start 124.46 35.56) (end 121.92 38.1) (width 0.25) (layer "F.Cu") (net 10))
 (segment (start 130.51 35.56) (end 124.46 35.56) (width 0.25) (layer "F.Cu") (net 10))
 (segment (start 120.896 39.124) (end 113.814 39.124) (width 0.25) (layer "B.Cu") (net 10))
 (segment (start 121.92 38.1) (end 120.896 39.124) (width 0.25) (layer "B.Cu") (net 10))
 (segment (start 113.814 39.124) (end 112.69 38) (width 0.25) (layer "B.Cu") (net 10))
 (segment (start 121.96 33.06) (end 121.92 33.02) (width 0.25) (layer "F.Cu") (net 6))
 (segment (start 130.51 33.06) (end 121.96 33.06) (width 0.25) (layer "F.Cu") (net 6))
 (segment (start 120.854 31.954) (end 113.656 31.954) (width 0.25) (layer "B.Cu") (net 6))
 (segment (start 113.656 31.954) (end 112.69 32.92) (width 0.25) (layer "B.Cu") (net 6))
 (segment (start 121.92 33.02) (end 120.854 31.954) (width 0.25) (layer "B.Cu") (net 6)))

